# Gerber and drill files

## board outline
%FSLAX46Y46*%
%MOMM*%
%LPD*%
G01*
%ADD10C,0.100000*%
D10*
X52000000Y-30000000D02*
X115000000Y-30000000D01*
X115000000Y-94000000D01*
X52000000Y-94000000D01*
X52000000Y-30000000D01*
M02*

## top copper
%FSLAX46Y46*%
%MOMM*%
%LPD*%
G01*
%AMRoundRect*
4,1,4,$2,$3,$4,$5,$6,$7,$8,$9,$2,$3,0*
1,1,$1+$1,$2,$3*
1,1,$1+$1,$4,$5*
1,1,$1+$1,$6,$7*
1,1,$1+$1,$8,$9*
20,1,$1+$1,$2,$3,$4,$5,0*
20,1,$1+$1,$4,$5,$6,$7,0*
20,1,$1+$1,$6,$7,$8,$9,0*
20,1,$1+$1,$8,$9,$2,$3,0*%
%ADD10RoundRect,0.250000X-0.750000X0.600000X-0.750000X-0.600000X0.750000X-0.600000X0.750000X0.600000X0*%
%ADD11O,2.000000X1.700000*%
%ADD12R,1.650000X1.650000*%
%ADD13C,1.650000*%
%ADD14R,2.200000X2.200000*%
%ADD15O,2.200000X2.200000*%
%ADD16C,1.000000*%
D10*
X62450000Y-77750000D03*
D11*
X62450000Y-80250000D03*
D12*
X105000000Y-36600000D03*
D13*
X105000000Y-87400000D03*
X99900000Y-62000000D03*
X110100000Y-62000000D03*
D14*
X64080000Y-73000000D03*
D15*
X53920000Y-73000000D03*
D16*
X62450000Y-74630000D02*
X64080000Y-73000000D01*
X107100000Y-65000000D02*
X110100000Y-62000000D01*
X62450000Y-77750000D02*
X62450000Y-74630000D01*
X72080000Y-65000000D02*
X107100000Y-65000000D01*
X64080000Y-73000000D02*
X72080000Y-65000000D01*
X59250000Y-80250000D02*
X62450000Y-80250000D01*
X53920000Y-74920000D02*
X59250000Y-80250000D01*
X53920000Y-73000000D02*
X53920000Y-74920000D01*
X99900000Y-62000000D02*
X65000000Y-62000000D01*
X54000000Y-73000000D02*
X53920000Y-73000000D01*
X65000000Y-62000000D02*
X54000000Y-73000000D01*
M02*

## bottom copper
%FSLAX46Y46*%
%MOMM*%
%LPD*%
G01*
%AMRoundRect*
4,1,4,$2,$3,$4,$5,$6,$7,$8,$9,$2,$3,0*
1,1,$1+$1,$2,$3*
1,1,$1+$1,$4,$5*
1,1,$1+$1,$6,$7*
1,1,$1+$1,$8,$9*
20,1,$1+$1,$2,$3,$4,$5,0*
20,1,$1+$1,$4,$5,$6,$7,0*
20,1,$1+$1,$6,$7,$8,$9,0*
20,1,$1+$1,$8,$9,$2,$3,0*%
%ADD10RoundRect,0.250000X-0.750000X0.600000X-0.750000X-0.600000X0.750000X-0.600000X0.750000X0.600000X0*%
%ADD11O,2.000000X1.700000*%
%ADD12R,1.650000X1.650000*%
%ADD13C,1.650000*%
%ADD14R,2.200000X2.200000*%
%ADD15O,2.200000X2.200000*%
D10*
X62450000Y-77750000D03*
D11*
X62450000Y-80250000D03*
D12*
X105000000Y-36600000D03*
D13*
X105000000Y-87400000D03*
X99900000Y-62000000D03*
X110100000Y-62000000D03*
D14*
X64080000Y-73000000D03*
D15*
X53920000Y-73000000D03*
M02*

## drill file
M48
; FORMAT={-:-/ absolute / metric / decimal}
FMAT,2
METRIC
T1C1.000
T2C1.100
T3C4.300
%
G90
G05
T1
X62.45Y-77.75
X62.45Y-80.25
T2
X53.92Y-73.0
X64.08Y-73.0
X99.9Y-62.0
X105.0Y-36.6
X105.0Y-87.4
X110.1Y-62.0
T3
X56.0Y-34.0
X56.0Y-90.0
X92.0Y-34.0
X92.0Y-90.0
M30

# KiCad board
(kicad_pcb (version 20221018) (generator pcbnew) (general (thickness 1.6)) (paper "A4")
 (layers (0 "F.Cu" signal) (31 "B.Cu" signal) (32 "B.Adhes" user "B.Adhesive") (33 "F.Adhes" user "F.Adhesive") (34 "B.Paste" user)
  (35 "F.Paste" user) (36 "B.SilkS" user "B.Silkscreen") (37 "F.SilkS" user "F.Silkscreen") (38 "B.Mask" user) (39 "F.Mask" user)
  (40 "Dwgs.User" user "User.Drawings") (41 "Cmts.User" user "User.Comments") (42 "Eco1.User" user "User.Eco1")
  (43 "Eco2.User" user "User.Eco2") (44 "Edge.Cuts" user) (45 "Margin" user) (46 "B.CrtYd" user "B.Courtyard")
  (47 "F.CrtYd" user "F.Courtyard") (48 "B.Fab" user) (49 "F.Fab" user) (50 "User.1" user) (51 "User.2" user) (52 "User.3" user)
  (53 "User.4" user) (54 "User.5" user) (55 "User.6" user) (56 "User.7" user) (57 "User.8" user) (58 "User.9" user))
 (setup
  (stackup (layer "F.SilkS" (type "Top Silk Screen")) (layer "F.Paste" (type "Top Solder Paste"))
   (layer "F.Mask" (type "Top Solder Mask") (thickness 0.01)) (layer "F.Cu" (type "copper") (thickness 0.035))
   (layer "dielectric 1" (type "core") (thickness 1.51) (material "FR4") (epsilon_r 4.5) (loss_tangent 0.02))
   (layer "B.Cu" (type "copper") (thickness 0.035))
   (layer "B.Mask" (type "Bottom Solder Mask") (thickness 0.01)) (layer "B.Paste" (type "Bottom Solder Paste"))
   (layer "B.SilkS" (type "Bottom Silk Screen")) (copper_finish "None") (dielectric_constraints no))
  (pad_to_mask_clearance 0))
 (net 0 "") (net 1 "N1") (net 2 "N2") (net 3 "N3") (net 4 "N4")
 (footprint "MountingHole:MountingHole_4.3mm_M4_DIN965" (layer "F.Cu") (at 92 34)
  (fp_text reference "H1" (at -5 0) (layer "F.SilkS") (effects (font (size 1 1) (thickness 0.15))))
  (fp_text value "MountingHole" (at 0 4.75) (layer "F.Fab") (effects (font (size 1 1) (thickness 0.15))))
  (pad "" np_thru_hole circle (at 0 0) (size 4.3 4.3) (drill 4.3) (layers "*.Cu" "*.Mask")))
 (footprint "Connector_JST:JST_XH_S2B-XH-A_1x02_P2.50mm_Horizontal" (layer "F.Cu") (at 62.45 77.75 -90)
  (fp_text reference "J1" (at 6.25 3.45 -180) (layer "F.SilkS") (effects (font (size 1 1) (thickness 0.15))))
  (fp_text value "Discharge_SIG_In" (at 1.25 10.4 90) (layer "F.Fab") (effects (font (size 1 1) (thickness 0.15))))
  (pad "1" thru_hole roundrect (at 0 0 270) (size 1.7 2) (drill 1) (layers "*.Cu" "*.Mask") (roundrect_rratio 0.147059) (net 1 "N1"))
  (pad "2" thru_hole oval (at 2.5 0 270) (size 1.7 2) (drill 1) (layers "*.Cu" "*.Mask") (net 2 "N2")))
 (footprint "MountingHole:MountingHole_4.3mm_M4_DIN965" (layer "F.Cu") (at 92 90)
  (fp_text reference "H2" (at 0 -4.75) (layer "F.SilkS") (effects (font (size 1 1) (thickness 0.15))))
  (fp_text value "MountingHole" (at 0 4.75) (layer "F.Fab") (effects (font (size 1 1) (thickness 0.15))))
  (pad "" np_thru_hole circle (at 0 0) (size 4.3 4.3) (drill 4.3) (layers "*.Cu" "*.Mask")))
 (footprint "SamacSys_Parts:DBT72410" (layer "F.Cu") (at 105 36.6 -90)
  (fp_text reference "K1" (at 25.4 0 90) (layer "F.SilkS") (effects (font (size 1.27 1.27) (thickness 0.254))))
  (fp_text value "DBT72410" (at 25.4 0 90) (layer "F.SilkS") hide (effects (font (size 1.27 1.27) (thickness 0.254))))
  (pad "1" thru_hole rect (at 0 0 270) (size 1.65 1.65) (drill 1.1) (layers "*.Cu" "*.Mask") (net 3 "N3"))
  (pad "2" thru_hole circle (at 50.8 0 270) (size 1.65 1.65) (drill 1.1) (layers "*.Cu" "*.Mask") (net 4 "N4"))
  (pad "3" thru_hole circle (at 25.4 5.1 270) (size 1.65 1.65) (drill 1.1) (layers "*.Cu" "*.Mask") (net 2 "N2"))
  (pad "4" thru_hole circle (at 25.4 -5.1 270) (size 1.65 1.65) (drill 1.1) (layers "*.Cu" "*.Mask") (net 1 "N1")))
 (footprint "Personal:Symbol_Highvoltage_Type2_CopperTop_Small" (layer "F.Cu") (at 83.3 51.505)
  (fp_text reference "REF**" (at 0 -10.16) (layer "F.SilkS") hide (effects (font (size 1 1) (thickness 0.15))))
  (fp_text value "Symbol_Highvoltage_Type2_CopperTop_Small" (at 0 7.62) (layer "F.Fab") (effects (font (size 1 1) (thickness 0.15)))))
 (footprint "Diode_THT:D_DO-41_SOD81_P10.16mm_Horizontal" (layer "F.Cu") (at 64.08 73 180)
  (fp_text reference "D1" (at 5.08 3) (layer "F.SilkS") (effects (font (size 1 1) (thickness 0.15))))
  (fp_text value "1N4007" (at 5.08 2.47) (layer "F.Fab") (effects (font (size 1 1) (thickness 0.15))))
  (pad "1" thru_hole rect (at 0 0 180) (size 2.2 2.2) (drill 1.1) (layers "*.Cu" "*.Mask") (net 1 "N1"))
  (pad "2" thru_hole oval (at 10.16 0 180) (size 2.2 2.2) (drill 1.1) (layers "*.Cu" "*.Mask") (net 2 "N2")))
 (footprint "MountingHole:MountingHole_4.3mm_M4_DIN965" (layer "F.Cu") (at 56 90)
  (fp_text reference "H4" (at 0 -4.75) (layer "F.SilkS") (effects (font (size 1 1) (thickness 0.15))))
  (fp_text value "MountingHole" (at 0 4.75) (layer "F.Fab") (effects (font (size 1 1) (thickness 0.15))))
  (pad "" np_thru_hole circle (at 0 0) (size 4.3 4.3) (drill 4.3) (layers "*.Cu" "*.Mask")))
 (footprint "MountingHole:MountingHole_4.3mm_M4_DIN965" (layer "F.Cu") (at 56 34)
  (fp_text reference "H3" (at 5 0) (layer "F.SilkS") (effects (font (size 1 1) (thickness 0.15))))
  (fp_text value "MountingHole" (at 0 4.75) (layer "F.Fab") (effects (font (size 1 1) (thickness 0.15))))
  (pad "" np_thru_hole circle (at 0 0) (size 4.3 4.3) (drill 4.3) (layers "*.Cu" "*.Mask")))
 (gr_rect (start 52 30) (end 115 94) (stroke (width 0.1) (type default)) (fill none) (layer "Edge.Cuts"))
 (segment (start 62.45 74.63) (end 64.08 73) (width 1) (layer "F.Cu") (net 1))
 (segment (start 107.1 65) (end 110.1 62) (width 1) (layer "F.Cu") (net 1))
 (segment (start 62.45 77.75) (end 62.45 74.63) (width 1) (layer "F.Cu") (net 1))
 (segment (start 72.08 65) (end 107.1 65) (width 1) (layer "F.Cu") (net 1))
 (segment (start 64.08 73) (end 72.08 65) (width 1) (layer "F.Cu") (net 1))
 (segment (start 59.25 80.25) (end 62.45 80.25) (width 1) (layer "F.Cu") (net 2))
 (segment (start 53.92 74.92) (end 59.25 80.25) (width 1) (layer "F.Cu") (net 2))
 (segment (start 53.92 73) (end 53.92 74.92) (width 1) (layer "F.Cu") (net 2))
 (segment (start 99.9 62) (end 65 62) (width 1) (layer "F.Cu") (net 2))
 (segment (start 54 73) (end 53.92 73) (width 1) (layer "F.Cu") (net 2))
 (segment (start 65 62) (end 54 73) (width 1) (layer "F.Cu") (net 2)))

